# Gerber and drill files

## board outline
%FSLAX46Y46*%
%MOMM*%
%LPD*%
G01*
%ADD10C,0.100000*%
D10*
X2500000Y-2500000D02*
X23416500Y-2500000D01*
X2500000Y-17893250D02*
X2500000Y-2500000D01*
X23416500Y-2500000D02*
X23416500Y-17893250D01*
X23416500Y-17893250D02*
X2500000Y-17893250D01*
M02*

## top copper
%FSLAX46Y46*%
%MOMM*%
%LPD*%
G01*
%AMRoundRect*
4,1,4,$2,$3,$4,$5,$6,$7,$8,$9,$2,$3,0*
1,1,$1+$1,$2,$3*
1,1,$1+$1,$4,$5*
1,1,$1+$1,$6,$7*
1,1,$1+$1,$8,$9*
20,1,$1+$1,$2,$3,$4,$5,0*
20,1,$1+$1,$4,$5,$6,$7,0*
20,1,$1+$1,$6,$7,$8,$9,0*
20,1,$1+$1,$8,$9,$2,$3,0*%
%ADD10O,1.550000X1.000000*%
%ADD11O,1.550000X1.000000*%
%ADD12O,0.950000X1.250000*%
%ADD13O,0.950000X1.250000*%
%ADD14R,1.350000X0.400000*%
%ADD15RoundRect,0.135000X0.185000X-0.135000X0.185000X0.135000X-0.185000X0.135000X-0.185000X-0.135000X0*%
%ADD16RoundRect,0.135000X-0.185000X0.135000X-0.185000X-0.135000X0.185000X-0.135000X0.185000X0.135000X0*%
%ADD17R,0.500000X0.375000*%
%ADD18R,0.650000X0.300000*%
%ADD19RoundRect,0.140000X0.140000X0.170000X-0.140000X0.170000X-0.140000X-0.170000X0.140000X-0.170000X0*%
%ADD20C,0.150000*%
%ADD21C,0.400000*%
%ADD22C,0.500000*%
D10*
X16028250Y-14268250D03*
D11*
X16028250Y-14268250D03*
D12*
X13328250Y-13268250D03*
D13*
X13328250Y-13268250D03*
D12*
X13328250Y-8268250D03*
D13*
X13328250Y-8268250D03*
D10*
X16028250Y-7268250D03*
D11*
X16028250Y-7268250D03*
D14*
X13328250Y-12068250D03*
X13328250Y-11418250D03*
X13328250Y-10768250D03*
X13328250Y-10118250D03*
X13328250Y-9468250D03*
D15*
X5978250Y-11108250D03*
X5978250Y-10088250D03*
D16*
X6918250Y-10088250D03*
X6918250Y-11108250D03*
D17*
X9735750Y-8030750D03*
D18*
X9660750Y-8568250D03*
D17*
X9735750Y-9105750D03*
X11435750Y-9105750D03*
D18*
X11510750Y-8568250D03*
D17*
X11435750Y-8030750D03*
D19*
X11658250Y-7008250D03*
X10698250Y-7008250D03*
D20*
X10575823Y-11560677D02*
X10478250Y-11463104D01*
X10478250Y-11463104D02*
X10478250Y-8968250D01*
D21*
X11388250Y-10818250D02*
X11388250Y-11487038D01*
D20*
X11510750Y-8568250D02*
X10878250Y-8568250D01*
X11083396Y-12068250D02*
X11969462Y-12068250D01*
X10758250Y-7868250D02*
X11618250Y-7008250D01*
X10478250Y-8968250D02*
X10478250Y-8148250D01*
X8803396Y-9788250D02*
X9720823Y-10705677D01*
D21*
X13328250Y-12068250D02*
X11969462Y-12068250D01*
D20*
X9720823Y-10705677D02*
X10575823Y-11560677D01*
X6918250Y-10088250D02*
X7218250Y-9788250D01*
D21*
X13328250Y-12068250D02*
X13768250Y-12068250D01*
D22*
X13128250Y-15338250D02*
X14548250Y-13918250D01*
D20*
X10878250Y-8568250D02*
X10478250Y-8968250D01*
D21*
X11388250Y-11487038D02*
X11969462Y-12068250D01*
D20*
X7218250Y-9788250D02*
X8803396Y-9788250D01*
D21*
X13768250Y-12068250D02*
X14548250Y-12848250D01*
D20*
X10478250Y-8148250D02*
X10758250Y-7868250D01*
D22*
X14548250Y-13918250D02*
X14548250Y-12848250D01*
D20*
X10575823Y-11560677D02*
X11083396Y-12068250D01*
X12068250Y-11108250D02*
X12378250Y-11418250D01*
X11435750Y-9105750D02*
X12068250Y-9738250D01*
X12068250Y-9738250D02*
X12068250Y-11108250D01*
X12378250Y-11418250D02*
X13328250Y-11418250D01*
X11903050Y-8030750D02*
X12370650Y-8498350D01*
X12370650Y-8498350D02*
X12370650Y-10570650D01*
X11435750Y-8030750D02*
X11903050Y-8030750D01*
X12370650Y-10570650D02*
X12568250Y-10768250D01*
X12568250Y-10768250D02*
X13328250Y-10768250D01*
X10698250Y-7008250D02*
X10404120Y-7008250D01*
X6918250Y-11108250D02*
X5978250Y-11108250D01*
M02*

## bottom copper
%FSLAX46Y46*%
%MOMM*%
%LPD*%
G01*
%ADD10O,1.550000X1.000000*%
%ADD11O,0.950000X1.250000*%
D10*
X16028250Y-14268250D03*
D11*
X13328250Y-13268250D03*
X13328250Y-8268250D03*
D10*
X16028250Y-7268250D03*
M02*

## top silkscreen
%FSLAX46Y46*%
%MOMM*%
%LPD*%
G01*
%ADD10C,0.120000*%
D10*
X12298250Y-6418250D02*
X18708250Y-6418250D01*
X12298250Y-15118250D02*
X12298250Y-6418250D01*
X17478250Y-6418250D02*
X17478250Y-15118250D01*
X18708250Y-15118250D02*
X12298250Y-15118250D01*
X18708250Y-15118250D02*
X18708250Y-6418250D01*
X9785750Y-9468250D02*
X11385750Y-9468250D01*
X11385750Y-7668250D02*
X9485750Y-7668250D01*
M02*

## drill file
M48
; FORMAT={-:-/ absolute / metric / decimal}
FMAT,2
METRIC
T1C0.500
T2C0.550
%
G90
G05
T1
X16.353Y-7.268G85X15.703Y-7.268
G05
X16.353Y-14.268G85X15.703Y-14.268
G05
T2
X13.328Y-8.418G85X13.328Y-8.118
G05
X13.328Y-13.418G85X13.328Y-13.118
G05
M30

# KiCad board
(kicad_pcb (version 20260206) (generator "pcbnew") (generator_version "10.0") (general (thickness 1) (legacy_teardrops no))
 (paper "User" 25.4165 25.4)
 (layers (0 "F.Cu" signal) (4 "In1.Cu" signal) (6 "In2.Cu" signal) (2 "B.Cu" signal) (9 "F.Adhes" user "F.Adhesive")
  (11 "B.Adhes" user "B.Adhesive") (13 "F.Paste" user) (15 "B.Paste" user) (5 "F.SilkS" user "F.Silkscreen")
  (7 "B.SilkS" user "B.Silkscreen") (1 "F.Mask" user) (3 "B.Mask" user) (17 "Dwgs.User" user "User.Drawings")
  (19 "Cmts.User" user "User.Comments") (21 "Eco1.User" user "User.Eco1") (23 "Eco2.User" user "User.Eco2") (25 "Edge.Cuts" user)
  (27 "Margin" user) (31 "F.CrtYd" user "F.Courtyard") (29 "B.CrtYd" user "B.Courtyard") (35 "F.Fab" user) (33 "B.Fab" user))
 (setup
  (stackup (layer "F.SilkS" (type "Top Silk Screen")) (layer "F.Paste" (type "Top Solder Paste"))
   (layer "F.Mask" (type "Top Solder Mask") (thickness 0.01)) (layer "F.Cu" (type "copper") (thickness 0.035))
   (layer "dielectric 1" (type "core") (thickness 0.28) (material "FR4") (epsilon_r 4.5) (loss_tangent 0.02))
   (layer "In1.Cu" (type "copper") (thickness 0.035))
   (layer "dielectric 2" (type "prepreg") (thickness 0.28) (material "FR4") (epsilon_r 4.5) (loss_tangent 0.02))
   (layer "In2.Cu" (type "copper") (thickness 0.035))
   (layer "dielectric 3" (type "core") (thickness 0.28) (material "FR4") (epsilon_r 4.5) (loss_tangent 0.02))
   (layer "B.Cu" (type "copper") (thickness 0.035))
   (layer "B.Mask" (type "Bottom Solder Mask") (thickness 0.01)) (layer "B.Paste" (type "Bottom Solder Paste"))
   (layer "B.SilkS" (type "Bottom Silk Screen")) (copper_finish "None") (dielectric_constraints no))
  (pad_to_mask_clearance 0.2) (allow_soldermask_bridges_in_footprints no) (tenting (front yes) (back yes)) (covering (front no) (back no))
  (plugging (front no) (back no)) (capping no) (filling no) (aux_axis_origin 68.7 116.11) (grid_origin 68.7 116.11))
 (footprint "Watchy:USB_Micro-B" (layer "F.Cu") (at 15.05825 10.76825 90)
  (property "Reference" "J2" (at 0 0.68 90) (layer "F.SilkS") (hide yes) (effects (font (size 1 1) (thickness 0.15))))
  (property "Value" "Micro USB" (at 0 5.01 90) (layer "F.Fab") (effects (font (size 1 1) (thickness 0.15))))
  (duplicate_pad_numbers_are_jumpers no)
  (fp_line (start 4.35 -2.76) (end 4.35 3.65) (stroke (width 0.12) (type solid)) (layer "F.SilkS"))
  (fp_line (start -4.35 -2.76) (end 4.35 -2.76) (stroke (width 0.12) (type solid)) (layer "F.SilkS"))
  (fp_line (start 4.35 2.42) (end -4.35 2.42) (stroke (width 0.12) (type solid)) (layer "F.SilkS"))
  (fp_line (start -4.35 3.65) (end -4.35 -2.76) (stroke (width 0.12) (type solid)) (layer "F.SilkS"))
  (fp_line (start -4.35 3.65) (end 4.35 3.65) (stroke (width 0.12) (type solid)) (layer "F.SilkS"))
  (pad "" thru_hole oval (at -3.5 0.97 180) (size 1.55 1) (drill oval 1.15 0.5) (layers "*.Cu" "*.Mask") (remove_unused_layers no))
  (pad "" smd oval (at -3.5 0.97 180) (size 1.55 1) (layers "F.Cu" "F.Mask" "F.Paste"))
  (pad "" thru_hole oval (at -2.5 -1.73 180) (size 0.95 1.25) (drill oval 0.55 0.85) (layers "*.Cu" "*.Mask") (remove_unused_layers no))
  (pad "" smd oval (at -2.5 -1.73 180) (size 0.95 1.25) (layers "F.Cu" "F.Mask" "F.Paste"))
  (pad "" thru_hole oval (at 2.5 -1.73 180) (size 0.95 1.25) (drill oval 0.55 0.85) (layers "*.Cu" "*.Mask") (remove_unused_layers no))
  (pad "" smd oval (at 2.5 -1.73 180) (size 0.95 1.25) (layers "F.Cu" "F.Mask" "F.Paste"))
  (pad "" thru_hole oval (at 3.5 0.97 180) (size 1.55 1) (drill oval 1.15 0.5) (layers "*.Cu" "*.Mask") (remove_unused_layers no))
  (pad "" smd oval (at 3.5 0.97 180) (size 1.55 1) (layers "F.Cu" "F.Mask" "F.Paste"))
  (pad "1" smd rect (at -1.3 -1.73 180) (size 1.35 0.4) (layers "F.Cu" "F.Mask" "F.Paste") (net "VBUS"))
  (pad "2" smd rect (at -0.65 -1.73 180) (size 1.35 0.4) (layers "F.Cu" "F.Mask" "F.Paste") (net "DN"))
  (pad "3" smd rect (at 0 -1.73 180) (size 1.35 0.4) (layers "F.Cu" "F.Mask" "F.Paste") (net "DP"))
  (pad "4" smd rect (at 0.65 -1.73 180) (size 1.35 0.4) (layers "F.Cu" "F.Mask" "F.Paste") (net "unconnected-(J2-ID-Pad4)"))
  (pad "5" smd rect (at 1.3 -1.73 180) (size 1.35 0.4) (layers "F.Cu" "F.Mask" "F.Paste") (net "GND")))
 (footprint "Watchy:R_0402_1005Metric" (layer "F.Cu") (at 5.97825 10.59825 90)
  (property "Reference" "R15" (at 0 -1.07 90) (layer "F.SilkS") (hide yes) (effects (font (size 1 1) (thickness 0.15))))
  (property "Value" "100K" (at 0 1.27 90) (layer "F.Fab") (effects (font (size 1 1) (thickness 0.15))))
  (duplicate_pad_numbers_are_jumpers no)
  (pad "1" smd roundrect (at -0.51 0 90) (size 0.54 0.64) (layers "F.Cu" "F.Mask" "F.Paste") (roundrect_rratio 0.25) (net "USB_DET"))
  (pad "2" smd roundrect (at 0.51 0 90) (size 0.54 0.64) (layers "F.Cu" "F.Mask" "F.Paste") (roundrect_rratio 0.25) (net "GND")))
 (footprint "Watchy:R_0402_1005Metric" (layer "F.Cu") (at 6.91825 10.59825 -90)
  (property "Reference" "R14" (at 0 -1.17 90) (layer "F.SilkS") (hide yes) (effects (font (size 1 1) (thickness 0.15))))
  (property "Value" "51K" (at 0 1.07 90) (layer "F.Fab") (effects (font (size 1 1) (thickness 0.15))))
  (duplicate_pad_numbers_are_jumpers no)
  (pad "1" smd roundrect (at -0.51 0 270) (size 0.54 0.64) (layers "F.Cu" "F.Mask" "F.Paste") (roundrect_rratio 0.25) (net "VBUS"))
  (pad "2" smd roundrect (at 0.51 0 270) (size 0.54 0.64) (layers "F.Cu" "F.Mask" "F.Paste") (roundrect_rratio 0.25) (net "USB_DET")))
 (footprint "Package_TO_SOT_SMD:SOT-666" (layer "F.Cu") (at 10.58575 8.56825)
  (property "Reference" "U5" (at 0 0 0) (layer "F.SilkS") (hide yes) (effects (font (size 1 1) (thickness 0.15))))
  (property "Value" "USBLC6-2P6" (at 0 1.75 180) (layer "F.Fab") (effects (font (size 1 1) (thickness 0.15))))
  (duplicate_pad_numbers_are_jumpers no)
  (fp_line (start -0.8 0.9) (end 0.8 0.9) (stroke (width 0.12) (type solid)) (layer "F.SilkS"))
  (fp_line (start 0.8 -0.9) (end -1.1 -0.9) (stroke (width 0.12) (type solid)) (layer "F.SilkS"))
  (pad "1" smd rect (at -0.85 -0.5375) (size 0.5 0.375) (layers "F.Cu" "F.Mask" "F.Paste") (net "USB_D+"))
  (pad "2" smd rect (at -0.925 0) (size 0.65 0.3) (layers "F.Cu" "F.Mask" "F.Paste") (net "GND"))
  (pad "3" smd rect (at -0.85 0.5375) (size 0.5 0.375) (layers "F.Cu" "F.Mask" "F.Paste") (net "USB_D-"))
  (pad "4" smd rect (at 0.85 0.5375) (size 0.5 0.375) (layers "F.Cu" "F.Mask" "F.Paste") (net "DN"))
  (pad "5" smd rect (at 0.925 0) (size 0.65 0.3) (layers "F.Cu" "F.Mask" "F.Paste") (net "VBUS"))
  (pad "6" smd rect (at 0.85 -0.5375) (size 0.5 0.375) (layers "F.Cu" "F.Mask" "F.Paste") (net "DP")))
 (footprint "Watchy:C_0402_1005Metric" (layer "F.Cu") (at 11.17825 7.00825 180)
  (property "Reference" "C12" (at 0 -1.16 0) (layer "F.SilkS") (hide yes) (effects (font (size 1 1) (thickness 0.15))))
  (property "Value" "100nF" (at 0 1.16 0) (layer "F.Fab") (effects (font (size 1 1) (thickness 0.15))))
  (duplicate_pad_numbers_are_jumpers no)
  (pad "1" smd roundrect (at -0.48 0 180) (size 0.56 0.62) (layers "F.Cu" "F.Mask" "F.Paste") (roundrect_rratio 0.25) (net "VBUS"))
  (pad "2" smd roundrect (at 0.48 0 180) (size 0.56 0.62) (layers "F.Cu" "F.Mask" "F.Paste") (roundrect_rratio 0.25) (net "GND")))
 (gr_line (start 2.5 2.5) (end 23.4165 2.5) (stroke (width 0.1) (type default)) (layer "Edge.Cuts"))
 (gr_line (start 2.5 17.89325) (end 2.5 2.5) (stroke (width 0.1) (type default)) (layer "Edge.Cuts"))
 (gr_line (start 23.4165 2.5) (end 23.4165 17.89325) (stroke (width 0.1) (type default)) (layer "Edge.Cuts"))
 (gr_line (start 23.4165 17.89325) (end 2.5 17.89325) (stroke (width 0.1) (type default)) (layer "Edge.Cuts"))
 (segment (start 10.575823 11.560677) (end 10.47825 11.463104) (width 0.15) (layer "F.Cu") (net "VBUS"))
 (segment (start 10.47825 11.463104) (end 10.47825 8.96825) (width 0.15) (layer "F.Cu") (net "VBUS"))
 (segment (start 11.38825 10.81825) (end 11.38825 11.487038) (width 0.4) (layer "F.Cu") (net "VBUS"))
 (segment (start 11.51075 8.56825) (end 10.87825 8.56825) (width 0.15) (layer "F.Cu") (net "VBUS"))
 (segment (start 11.083396 12.06825) (end 11.969462 12.06825) (width 0.15) (layer "F.Cu") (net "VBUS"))
 (segment (start 10.75825 7.86825) (end 11.61825 7.00825) (width 0.15) (layer "F.Cu") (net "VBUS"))
 (segment (start 10.47825 8.96825) (end 10.47825 8.14825) (width 0.15) (layer "F.Cu") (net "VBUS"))
 (segment (start 8.803396 9.78825) (end 9.720823 10.705677) (width 0.15) (layer "F.Cu") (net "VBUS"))
 (segment (start 13.32825 12.06825) (end 11.969462 12.06825) (width 0.4) (layer "F.Cu") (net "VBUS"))
 (segment (start 9.720823 10.705677) (end 10.575823 11.560677) (width 0.15) (layer "F.Cu") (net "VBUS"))
 (segment (start 6.91825 10.08825) (end 7.21825 9.78825) (width 0.15) (layer "F.Cu") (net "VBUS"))
 (segment (start 13.32825 12.06825) (end 13.76825 12.06825) (width 0.4) (layer "F.Cu") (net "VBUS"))
 (segment (start 13.12825 15.33825) (end 14.54825 13.91825) (width 0.5) (layer "F.Cu") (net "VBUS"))
 (segment (start 10.87825 8.56825) (end 10.47825 8.96825) (width 0.15) (layer "F.Cu") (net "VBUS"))
 (segment (start 11.38825 11.487038) (end 11.969462 12.06825) (width 0.4) (layer "F.Cu") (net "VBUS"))
 (segment (start 7.21825 9.78825) (end 8.803396 9.78825) (width 0.15) (layer "F.Cu") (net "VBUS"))
 (segment (start 13.76825 12.06825) (end 14.54825 12.84825) (width 0.4) (layer "F.Cu") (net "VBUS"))
 (segment (start 10.47825 8.14825) (end 10.75825 7.86825) (width 0.15) (layer "F.Cu") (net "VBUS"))
 (segment (start 14.54825 13.91825) (end 14.54825 12.84825) (width 0.5) (layer "F.Cu") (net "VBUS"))
 (segment (start 10.575823 11.560677) (end 11.083396 12.06825) (width 0.15) (layer "F.Cu") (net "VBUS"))
 (segment (start 12.06825 11.10825) (end 12.37825 11.41825) (width 0.15) (layer "F.Cu") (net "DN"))
 (segment (start 11.43575 9.10575) (end 12.06825 9.73825) (width 0.15) (layer "F.Cu") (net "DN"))
 (segment (start 12.06825 9.73825) (end 12.06825 11.10825) (width 0.15) (layer "F.Cu") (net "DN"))
 (segment (start 12.37825 11.41825) (end 13.32825 11.41825) (width 0.15) (layer "F.Cu") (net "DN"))
 (segment (start 11.90305 8.03075) (end 12.37065 8.49835) (width 0.15) (layer "F.Cu") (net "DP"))
 (segment (start 12.37065 8.49835) (end 12.37065 10.57065) (width 0.15) (layer "F.Cu") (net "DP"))
 (segment (start 11.43575 8.03075) (end 11.90305 8.03075) (width 0.15) (layer "F.Cu") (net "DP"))
 (segment (start 12.37065 10.57065) (end 12.56825 10.76825) (width 0.15) (layer "F.Cu") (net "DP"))
 (segment (start 12.56825 10.76825) (end 13.32825 10.76825) (width 0.15) (layer "F.Cu") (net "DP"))
 (segment (start 10.69825 7.00825) (end 10.40412 7.00825) (width 0.15) (layer "F.Cu") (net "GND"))
 (segment (start 6.91825 11.10825) (end 5.97825 11.10825) (width 0.15) (layer "F.Cu") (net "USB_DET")))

